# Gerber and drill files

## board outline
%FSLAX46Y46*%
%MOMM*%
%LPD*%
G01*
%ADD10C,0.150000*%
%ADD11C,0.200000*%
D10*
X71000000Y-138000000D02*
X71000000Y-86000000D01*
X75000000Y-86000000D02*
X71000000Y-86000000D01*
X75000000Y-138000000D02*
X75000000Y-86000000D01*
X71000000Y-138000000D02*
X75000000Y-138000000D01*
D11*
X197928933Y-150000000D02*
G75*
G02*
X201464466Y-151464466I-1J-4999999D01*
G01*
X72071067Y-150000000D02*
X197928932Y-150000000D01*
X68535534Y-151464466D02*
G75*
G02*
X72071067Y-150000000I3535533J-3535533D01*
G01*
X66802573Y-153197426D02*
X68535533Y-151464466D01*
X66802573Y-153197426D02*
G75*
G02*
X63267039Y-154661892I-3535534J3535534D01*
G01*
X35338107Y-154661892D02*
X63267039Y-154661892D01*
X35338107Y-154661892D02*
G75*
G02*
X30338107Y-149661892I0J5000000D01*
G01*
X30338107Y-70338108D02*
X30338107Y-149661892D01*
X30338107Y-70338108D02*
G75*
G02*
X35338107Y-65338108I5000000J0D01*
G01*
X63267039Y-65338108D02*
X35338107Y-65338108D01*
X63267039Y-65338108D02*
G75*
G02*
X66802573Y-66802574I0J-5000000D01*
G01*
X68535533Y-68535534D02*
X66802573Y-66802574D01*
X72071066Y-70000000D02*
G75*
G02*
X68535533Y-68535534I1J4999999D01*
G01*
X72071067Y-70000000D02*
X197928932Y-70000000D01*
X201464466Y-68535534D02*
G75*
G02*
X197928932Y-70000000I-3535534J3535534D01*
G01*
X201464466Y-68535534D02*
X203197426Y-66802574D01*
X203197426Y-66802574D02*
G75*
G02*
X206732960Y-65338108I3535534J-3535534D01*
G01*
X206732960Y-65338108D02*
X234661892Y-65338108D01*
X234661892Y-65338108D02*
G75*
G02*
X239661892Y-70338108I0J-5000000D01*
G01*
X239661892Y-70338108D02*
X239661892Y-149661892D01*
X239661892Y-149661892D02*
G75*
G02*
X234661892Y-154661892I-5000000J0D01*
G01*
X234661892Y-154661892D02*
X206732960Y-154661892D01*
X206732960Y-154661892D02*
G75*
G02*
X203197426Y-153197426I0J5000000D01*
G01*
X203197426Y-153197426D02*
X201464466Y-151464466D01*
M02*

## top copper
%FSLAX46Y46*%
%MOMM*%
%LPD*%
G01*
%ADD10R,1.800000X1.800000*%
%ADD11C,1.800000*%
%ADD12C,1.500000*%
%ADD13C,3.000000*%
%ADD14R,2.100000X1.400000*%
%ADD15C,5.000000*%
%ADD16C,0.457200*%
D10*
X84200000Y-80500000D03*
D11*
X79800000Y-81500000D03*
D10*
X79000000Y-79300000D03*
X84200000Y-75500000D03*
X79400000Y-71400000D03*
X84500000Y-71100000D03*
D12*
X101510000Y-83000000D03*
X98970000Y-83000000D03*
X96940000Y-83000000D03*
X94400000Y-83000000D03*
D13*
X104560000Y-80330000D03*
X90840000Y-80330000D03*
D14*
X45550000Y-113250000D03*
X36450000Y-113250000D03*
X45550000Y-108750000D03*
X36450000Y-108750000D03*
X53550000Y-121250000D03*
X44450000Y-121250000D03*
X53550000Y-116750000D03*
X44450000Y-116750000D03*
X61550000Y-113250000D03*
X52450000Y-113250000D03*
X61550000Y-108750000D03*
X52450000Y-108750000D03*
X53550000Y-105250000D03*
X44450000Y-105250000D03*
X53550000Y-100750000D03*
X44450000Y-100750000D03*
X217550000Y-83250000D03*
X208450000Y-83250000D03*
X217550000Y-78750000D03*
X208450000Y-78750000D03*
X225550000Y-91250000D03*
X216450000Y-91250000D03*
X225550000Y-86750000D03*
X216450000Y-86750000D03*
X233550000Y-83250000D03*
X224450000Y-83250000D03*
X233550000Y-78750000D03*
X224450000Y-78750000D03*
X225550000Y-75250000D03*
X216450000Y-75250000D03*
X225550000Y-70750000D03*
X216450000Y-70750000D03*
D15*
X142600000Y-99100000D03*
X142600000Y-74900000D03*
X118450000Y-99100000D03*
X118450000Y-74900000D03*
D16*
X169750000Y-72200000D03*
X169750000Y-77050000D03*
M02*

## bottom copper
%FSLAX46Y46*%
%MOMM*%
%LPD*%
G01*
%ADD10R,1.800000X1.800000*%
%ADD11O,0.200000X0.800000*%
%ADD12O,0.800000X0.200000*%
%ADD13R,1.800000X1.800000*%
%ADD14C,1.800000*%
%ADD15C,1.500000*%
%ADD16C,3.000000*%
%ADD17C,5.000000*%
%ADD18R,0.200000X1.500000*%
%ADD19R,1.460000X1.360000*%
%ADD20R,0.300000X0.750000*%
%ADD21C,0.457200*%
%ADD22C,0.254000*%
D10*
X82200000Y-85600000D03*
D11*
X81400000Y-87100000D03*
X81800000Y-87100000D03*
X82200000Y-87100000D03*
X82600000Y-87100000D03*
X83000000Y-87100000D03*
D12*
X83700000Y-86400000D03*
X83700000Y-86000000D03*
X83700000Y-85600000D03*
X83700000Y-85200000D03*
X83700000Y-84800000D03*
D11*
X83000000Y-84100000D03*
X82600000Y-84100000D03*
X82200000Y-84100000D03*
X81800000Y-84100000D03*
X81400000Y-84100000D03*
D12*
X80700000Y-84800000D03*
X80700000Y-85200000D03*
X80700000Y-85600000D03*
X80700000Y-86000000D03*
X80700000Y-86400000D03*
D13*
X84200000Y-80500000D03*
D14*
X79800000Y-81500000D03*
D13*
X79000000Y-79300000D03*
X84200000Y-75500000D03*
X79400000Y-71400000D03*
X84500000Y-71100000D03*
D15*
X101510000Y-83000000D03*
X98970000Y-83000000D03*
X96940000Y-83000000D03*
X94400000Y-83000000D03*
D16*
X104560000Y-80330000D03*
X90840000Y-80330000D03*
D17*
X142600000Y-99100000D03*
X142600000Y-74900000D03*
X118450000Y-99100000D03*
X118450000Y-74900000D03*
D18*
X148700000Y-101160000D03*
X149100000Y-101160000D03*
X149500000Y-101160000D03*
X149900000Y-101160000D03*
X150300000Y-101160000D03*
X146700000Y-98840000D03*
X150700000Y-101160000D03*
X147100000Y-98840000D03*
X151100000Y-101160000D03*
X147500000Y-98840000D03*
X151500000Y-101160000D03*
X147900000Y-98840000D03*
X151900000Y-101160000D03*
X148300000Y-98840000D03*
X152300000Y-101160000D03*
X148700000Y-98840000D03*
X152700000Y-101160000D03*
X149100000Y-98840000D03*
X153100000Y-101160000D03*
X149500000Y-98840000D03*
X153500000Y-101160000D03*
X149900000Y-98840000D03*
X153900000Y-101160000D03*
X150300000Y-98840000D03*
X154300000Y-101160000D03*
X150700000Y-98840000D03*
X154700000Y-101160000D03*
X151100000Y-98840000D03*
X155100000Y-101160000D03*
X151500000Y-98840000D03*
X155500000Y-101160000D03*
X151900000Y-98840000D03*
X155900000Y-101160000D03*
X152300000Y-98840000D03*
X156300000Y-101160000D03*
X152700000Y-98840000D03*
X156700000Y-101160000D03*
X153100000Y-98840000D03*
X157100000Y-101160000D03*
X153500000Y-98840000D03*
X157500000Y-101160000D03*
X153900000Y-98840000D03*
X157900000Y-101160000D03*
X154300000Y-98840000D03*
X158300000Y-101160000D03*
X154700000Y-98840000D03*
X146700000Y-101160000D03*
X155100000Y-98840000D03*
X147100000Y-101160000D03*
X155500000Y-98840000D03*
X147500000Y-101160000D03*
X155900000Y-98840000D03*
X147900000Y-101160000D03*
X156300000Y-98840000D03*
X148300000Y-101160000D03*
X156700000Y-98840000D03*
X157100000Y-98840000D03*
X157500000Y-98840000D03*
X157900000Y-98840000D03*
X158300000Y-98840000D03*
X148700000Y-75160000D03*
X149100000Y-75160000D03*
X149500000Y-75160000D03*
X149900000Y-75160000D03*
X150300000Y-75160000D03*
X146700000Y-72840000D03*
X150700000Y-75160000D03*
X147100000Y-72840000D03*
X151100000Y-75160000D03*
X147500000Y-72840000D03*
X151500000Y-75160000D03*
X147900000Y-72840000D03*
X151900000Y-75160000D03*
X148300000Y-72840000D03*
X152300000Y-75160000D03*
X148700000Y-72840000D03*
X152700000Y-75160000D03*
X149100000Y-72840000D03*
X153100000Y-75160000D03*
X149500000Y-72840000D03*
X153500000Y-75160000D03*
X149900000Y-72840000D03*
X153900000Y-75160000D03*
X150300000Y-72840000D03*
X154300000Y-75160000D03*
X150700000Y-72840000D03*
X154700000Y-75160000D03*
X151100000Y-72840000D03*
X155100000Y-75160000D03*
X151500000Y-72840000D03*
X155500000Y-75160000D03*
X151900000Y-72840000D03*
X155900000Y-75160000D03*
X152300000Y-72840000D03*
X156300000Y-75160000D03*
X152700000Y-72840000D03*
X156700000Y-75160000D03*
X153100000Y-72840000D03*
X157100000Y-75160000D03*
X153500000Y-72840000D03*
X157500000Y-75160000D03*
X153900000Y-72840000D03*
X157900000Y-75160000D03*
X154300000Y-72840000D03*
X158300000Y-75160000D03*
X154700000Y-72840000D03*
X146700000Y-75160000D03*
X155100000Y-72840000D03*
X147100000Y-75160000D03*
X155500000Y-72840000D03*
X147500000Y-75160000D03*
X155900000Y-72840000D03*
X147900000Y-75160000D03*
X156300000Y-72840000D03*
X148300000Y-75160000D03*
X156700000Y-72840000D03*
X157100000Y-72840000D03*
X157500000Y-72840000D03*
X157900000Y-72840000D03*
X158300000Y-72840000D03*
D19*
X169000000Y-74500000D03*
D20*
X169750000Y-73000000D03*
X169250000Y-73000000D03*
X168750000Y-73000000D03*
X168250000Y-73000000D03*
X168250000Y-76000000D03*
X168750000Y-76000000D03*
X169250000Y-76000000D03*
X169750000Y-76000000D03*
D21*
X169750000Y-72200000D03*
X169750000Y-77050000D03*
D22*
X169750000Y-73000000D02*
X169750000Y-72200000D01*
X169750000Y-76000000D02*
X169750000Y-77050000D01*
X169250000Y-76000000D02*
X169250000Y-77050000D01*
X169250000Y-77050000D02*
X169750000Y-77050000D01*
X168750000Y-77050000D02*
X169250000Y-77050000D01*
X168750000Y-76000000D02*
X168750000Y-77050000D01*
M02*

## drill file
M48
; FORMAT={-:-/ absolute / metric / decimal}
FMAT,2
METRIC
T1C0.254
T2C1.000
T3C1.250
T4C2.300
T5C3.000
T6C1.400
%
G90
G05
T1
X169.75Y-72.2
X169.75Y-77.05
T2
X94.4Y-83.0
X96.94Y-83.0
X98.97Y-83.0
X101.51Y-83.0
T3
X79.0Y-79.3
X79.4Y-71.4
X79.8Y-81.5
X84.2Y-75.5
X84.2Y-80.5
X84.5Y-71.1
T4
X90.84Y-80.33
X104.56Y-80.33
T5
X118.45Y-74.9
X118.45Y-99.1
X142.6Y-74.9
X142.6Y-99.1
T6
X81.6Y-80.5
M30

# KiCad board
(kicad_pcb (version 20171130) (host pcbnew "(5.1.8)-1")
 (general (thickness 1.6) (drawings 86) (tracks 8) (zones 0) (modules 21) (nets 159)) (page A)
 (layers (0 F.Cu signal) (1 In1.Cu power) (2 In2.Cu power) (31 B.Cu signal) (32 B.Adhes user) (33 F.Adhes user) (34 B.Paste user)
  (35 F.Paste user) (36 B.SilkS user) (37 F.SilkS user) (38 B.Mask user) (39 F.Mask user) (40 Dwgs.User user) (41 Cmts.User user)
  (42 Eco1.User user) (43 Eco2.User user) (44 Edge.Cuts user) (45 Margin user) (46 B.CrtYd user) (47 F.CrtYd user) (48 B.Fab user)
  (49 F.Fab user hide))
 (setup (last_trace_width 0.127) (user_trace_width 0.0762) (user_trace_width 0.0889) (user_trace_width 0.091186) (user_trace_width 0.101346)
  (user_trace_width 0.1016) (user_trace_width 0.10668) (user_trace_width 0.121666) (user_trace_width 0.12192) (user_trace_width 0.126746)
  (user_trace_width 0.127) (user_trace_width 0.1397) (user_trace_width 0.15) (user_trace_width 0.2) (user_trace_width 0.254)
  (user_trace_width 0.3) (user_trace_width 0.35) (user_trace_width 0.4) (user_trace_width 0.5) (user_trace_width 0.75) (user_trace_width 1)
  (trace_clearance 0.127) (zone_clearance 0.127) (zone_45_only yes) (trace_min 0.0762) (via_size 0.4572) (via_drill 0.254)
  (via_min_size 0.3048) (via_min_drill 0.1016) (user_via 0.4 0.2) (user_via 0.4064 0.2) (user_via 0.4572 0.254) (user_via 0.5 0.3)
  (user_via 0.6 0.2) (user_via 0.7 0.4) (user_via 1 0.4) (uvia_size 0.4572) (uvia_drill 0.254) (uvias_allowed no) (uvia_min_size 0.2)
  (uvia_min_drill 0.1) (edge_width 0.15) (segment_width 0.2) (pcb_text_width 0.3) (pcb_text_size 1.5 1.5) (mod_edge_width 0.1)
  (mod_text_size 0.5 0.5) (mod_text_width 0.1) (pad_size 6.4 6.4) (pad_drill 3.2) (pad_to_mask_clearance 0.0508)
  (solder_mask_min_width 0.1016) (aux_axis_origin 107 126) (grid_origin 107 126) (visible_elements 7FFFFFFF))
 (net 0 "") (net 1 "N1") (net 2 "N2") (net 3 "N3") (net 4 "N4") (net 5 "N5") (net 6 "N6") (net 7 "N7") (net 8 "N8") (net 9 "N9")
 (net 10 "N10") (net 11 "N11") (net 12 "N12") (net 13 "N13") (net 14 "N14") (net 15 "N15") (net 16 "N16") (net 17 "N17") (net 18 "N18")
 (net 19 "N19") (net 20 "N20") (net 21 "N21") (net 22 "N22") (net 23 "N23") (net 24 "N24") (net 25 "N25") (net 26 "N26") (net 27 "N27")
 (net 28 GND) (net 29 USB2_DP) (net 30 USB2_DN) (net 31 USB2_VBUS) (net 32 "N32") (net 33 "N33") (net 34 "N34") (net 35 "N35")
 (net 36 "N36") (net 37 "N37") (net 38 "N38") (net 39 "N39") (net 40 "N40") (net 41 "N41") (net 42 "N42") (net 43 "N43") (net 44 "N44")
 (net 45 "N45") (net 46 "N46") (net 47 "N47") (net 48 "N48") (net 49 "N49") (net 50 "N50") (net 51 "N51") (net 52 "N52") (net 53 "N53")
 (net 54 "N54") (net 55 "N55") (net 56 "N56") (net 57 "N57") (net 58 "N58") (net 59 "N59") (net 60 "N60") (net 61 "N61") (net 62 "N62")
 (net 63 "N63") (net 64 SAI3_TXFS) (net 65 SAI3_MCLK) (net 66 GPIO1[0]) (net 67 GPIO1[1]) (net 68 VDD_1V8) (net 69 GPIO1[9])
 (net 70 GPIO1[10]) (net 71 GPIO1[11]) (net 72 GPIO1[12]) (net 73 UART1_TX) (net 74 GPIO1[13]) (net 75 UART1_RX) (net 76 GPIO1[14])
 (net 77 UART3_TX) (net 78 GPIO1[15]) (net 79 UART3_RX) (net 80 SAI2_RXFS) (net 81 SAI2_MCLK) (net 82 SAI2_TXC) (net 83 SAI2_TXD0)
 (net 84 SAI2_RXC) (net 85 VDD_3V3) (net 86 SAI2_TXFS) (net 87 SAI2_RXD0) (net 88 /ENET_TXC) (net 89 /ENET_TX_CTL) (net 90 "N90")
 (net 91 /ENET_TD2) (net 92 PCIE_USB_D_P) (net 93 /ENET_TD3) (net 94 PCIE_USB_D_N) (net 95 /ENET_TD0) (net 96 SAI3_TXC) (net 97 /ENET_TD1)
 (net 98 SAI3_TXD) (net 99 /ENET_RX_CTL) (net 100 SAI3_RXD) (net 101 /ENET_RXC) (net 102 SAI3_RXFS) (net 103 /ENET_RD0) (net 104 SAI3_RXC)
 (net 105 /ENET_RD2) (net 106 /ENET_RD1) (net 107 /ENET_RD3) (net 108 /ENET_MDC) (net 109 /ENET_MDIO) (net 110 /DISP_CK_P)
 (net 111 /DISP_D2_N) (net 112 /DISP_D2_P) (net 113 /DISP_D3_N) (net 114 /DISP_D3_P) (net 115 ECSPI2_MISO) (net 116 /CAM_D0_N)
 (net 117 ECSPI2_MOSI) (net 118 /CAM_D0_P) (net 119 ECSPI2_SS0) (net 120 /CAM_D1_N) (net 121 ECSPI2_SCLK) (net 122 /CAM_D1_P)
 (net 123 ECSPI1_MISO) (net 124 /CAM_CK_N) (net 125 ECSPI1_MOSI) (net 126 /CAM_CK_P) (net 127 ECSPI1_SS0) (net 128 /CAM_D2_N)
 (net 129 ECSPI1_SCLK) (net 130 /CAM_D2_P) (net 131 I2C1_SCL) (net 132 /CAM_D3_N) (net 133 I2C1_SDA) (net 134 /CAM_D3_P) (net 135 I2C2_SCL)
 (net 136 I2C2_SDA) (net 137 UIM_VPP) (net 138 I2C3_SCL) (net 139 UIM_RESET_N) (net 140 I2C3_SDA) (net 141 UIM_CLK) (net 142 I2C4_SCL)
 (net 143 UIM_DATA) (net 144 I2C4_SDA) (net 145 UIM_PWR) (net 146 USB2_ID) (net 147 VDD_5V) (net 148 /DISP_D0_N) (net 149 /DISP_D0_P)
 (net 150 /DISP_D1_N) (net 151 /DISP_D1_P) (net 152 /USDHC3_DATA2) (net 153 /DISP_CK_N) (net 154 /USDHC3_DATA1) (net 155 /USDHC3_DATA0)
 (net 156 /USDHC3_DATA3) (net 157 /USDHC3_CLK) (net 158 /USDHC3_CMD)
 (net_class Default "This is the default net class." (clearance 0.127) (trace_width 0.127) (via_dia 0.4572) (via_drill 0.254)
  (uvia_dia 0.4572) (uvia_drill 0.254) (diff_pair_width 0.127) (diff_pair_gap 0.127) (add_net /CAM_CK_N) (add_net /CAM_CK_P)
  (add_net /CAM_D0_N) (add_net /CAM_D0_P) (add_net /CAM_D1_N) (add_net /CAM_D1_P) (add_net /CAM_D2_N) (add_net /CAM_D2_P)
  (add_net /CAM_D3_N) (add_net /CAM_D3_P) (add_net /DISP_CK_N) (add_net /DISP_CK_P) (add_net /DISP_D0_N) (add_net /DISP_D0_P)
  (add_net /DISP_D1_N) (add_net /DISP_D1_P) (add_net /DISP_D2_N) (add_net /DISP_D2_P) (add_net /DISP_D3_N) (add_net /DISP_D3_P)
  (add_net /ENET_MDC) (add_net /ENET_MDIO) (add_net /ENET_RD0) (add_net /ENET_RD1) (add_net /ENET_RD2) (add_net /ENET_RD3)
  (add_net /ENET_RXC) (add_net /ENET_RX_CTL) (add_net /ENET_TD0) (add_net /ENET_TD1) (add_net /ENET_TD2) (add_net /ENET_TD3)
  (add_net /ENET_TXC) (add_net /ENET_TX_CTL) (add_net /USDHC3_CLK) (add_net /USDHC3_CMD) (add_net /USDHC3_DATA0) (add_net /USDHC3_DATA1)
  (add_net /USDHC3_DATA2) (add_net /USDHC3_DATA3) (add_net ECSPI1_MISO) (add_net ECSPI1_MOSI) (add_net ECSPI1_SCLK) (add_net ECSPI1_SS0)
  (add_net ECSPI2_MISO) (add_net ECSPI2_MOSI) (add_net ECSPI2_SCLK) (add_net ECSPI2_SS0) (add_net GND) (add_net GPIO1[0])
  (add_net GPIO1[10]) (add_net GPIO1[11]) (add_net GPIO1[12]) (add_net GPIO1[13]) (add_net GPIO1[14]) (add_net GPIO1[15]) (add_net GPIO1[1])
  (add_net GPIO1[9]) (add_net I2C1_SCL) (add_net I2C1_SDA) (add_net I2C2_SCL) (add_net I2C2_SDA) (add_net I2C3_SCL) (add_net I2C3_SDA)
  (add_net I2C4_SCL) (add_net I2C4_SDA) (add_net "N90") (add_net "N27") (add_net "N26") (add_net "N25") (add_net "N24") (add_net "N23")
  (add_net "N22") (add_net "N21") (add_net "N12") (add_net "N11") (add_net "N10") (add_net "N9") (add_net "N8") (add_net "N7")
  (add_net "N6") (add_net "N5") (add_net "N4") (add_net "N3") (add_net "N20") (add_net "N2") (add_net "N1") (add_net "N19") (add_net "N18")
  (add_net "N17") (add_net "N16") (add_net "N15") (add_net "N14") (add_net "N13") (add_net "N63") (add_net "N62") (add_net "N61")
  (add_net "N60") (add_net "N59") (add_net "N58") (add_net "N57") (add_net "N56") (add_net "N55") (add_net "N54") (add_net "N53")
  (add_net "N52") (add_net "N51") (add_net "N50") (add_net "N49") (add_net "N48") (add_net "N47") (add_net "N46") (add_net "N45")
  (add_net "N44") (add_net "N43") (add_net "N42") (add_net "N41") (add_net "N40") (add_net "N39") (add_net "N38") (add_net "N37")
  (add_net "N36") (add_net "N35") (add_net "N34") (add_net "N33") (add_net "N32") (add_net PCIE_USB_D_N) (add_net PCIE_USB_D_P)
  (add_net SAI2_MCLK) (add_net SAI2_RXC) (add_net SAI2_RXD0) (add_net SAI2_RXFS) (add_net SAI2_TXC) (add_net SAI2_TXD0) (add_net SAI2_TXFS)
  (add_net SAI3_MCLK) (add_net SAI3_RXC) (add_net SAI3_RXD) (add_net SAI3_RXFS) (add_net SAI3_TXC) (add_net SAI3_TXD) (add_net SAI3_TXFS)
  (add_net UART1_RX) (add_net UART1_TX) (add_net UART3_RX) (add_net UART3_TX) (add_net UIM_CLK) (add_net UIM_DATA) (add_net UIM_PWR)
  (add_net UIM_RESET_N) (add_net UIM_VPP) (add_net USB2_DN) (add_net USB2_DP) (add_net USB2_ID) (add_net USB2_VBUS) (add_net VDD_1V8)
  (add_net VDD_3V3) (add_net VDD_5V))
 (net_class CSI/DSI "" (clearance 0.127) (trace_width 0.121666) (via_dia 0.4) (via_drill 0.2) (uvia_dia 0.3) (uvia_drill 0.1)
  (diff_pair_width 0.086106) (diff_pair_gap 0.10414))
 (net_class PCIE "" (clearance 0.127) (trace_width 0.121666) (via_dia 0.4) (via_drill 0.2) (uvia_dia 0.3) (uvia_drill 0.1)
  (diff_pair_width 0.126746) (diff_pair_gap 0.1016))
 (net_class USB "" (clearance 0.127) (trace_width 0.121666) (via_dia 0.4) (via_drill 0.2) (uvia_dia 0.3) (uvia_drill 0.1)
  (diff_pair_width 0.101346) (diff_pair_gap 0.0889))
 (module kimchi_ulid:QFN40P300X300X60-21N (layer B.Cu) (at 82.2 85.6)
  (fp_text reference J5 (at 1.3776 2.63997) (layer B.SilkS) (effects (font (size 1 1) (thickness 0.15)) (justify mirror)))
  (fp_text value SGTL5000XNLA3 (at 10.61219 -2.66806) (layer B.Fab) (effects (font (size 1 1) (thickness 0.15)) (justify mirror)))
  (pad 21 smd rect (at 0 0) (size 1.8 1.8) (layers B.Cu B.Mask) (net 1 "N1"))
  (pad 20 smd oval (at -0.8 1.5) (size 0.2 0.8) (layers B.Cu B.Paste B.Mask) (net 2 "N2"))
  (pad 19 smd oval (at -0.4 1.5) (size 0.2 0.8) (layers B.Cu B.Paste B.Mask) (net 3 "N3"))
  (pad 18 smd oval (at 0 1.5) (size 0.2 0.8) (layers B.Cu B.Paste B.Mask) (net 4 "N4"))
  (pad 17 smd oval (at 0.4 1.5) (size 0.2 0.8) (layers B.Cu B.Paste B.Mask) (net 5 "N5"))
  (pad 16 smd oval (at 0.8 1.5) (size 0.2 0.8) (layers B.Cu B.Paste B.Mask) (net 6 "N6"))
  (pad 15 smd oval (at 1.5 0.8) (size 0.8 0.2) (layers B.Cu B.Paste B.Mask) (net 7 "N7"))
  (pad 14 smd oval (at 1.5 0.4) (size 0.8 0.2) (layers B.Cu B.Paste B.Mask) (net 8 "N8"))
  (pad 13 smd oval (at 1.5 0) (size 0.8 0.2) (layers B.Cu B.Paste B.Mask) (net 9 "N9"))
  (pad 12 smd oval (at 1.5 -0.4) (size 0.8 0.2) (layers B.Cu B.Paste B.Mask) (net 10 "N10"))
  (pad 11 smd oval (at 1.5 -0.8) (size 0.8 0.2) (layers B.Cu B.Paste B.Mask) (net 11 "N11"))
  (pad 10 smd oval (at 0.8 -1.5) (size 0.2 0.8) (layers B.Cu B.Paste B.Mask) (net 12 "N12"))
  (pad 9 smd oval (at 0.4 -1.5) (size 0.2 0.8) (layers B.Cu B.Paste B.Mask) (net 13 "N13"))
  (pad 8 smd oval (at 0 -1.5) (size 0.2 0.8) (layers B.Cu B.Paste B.Mask) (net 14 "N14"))
  (pad 7 smd oval (at -0.4 -1.5) (size 0.2 0.8) (layers B.Cu B.Paste B.Mask) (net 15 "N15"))
  (pad 6 smd oval (at -0.8 -1.5) (size 0.2 0.8) (layers B.Cu B.Paste B.Mask) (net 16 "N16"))
  (pad 5 smd oval (at -1.5 -0.8) (size 0.8 0.2) (layers B.Cu B.Paste B.Mask) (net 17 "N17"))
  (pad 4 smd oval (at -1.5 -0.4) (size 0.8 0.2) (layers B.Cu B.Paste B.Mask) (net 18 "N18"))
  (pad 3 smd oval (at -1.5 0) (size 0.8 0.2) (layers B.Cu B.Paste B.Mask) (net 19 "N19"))
  (pad 2 smd oval (at -1.5 0.4) (size 0.8 0.2) (layers B.Cu B.Paste B.Mask) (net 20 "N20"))
  (pad 1 smd oval (at -1.5 0.8) (size 0.8 0.2) (layers B.Cu B.Paste B.Mask) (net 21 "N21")))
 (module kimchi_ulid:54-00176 (layer B.Cu) (at 81.6 70 270)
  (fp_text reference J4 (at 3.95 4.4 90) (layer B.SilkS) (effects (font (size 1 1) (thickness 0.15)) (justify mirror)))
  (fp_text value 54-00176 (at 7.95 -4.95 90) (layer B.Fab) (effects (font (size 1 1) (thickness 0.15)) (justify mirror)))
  (pad "" np_thru_hole circle (at 10.5 0 270) (size 1.4 1.4) (drill 1.4) (layers *.Cu *.Mask))
  (pad 6 thru_hole rect (at 10.5 -2.6 270) (size 1.8 1.8) (drill 1.25) (layers *.Cu *.Mask) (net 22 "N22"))
  (pad 5 thru_hole circle (at 11.5 1.8 270) (size 1.8 1.8) (drill 1.25) (layers *.Cu *.Mask) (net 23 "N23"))
  (pad 4 thru_hole rect (at 9.3 2.6 270) (size 1.8 1.8) (drill 1.25) (layers *.Cu *.Mask) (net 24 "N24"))
  (pad 3 thru_hole rect (at 5.5 -2.6 270) (size 1.8 1.8) (drill 1.25) (layers *.Cu *.Mask) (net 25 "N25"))
  (pad 2 thru_hole rect (at 1.4 2.2 270) (size 1.8 1.8) (drill 1.25) (layers *.Cu *.Mask) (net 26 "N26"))
  (pad 1 thru_hole rect (at 1.1 -2.9 270) (size 1.8 1.8) (drill 1.25) (layers *.Cu *.Mask) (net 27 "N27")))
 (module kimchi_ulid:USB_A (layer B.Cu) (at 94.4 83)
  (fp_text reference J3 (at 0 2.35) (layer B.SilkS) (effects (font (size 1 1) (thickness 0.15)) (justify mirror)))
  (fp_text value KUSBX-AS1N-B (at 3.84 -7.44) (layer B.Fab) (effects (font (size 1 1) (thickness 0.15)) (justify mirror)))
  (pad 4 thru_hole circle (at 7.11 0 90) (size 1.5 1.5) (drill 1) (layers *.Cu *.Mask) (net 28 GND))
  (pad 3 thru_hole circle (at 4.57 0 90) (size 1.5 1.5) (drill 1) (layers *.Cu *.Mask) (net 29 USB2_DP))
  (pad 2 thru_hole circle (at 2.54 0 90) (size 1.5 1.5) (drill 1) (layers *.Cu *.Mask) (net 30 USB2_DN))
  (pad 1 thru_hole circle (at 0 0 90) (size 1.5 1.5) (drill 1) (layers *.Cu *.Mask) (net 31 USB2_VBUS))
  (pad 5 thru_hole circle (at 10.16 -2.67 90) (size 3 3) (drill 2.3) (layers *.Cu *.Mask) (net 28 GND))
  (pad 5 thru_hole circle (at -3.56 -2.67 90) (size 3 3) (drill 2.3) (layers *.Cu *.Mask) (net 28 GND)))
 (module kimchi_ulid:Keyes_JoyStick (layer F.Cu) (at 221 111 180)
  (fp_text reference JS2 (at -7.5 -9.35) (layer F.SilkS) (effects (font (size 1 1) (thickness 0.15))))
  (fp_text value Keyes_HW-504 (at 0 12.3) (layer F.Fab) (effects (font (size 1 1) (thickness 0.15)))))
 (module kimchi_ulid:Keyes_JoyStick (layer F.Cu) (at 48.8 81)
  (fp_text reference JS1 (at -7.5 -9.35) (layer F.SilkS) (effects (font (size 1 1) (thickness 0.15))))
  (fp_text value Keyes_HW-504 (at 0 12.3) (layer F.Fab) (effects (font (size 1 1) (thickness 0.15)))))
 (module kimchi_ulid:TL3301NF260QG (layer F.Cu) (at 41 111)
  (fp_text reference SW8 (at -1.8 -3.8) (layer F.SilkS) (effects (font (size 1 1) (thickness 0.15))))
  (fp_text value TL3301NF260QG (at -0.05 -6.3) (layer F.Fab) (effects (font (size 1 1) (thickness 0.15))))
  (pad 4 smd rect (at 4.55 2.25) (size 2.1 1.4) (layers F.Cu F.Paste F.Mask) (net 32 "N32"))
  (pad 3 smd rect (at -4.55 2.25) (size 2.1 1.4) (layers F.Cu F.Paste F.Mask) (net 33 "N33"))
  (pad 2 smd rect (at 4.55 -2.25) (size 2.1 1.4) (layers F.Cu F.Paste F.Mask) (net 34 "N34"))
  (pad 1 smd rect (at -4.55 -2.25) (size 2.1 1.4) (layers F.Cu F.Paste F.Mask) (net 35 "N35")))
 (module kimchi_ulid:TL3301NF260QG (layer F.Cu) (at 49 119)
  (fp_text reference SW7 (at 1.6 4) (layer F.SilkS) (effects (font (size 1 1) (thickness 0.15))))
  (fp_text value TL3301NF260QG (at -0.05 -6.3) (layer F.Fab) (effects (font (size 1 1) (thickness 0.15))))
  (pad 4 smd rect (at 4.55 2.25) (size 2.1 1.4) (layers F.Cu F.Paste F.Mask) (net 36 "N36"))
  (pad 3 smd rect (at -4.55 2.25) (size 2.1 1.4) (layers F.Cu F.Paste F.Mask) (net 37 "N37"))
  (pad 2 smd rect (at 4.55 -2.25) (size 2.1 1.4) (layers F.Cu F.Paste F.Mask) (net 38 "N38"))
  (pad 1 smd rect (at -4.55 -2.25) (size 2.1 1.4) (layers F.Cu F.Paste F.Mask) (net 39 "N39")))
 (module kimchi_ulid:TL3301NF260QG (layer F.Cu) (at 57 111)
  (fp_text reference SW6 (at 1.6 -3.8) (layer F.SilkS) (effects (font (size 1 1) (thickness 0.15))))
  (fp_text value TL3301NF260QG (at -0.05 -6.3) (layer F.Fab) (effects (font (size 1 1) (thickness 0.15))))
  (pad 4 smd rect (at 4.55 2.25) (size 2.1 1.4) (layers F.Cu F.Paste F.Mask) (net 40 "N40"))
  (pad 3 smd rect (at -4.55 2.25) (size 2.1 1.4) (layers F.Cu F.Paste F.Mask) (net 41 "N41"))
  (pad 2 smd rect (at 4.55 -2.25) (size 2.1 1.4) (layers F.Cu F.Paste F.Mask) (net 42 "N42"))
  (pad 1 smd rect (at -4.55 -2.25) (size 2.1 1.4) (layers F.Cu F.Paste F.Mask) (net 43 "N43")))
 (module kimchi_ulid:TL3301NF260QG (layer F.Cu) (at 49 103)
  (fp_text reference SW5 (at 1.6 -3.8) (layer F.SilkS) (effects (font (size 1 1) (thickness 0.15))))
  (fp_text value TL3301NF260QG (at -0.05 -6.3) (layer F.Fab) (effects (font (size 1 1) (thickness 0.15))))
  (pad 4 smd rect (at 4.55 2.25) (size 2.1 1.4) (layers F.Cu F.Paste F.Mask) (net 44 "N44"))
  (pad 3 smd rect (at -4.55 2.25) (size 2.1 1.4) (layers F.Cu F.Paste F.Mask) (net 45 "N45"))
  (pad 2 smd rect (at 4.55 -2.25) (size 2.1 1.4) (layers F.Cu F.Paste F.Mask) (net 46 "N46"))
  (pad 1 smd rect (at -4.55 -2.25) (size 2.1 1.4) (layers F.Cu F.Paste F.Mask) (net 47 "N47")))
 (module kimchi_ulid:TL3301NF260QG (layer F.Cu) (at 213 81)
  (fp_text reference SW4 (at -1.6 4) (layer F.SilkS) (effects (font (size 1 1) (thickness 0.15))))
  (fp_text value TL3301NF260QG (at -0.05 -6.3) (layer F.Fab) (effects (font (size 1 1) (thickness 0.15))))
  (pad 4 smd rect (at 4.55 2.25) (size 2.1 1.4) (layers F.Cu F.Paste F.Mask) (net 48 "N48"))
  (pad 3 smd rect (at -4.55 2.25) (size 2.1 1.4) (layers F.Cu F.Paste F.Mask) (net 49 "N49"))
  (pad 2 smd rect (at 4.55 -2.25) (size 2.1 1.4) (layers F.Cu F.Paste F.Mask) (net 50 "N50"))
  (pad 1 smd rect (at -4.55 -2.25) (size 2.1 1.4) (layers F.Cu F.Paste F.Mask) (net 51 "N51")))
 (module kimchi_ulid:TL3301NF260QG (layer F.Cu) (at 221 89)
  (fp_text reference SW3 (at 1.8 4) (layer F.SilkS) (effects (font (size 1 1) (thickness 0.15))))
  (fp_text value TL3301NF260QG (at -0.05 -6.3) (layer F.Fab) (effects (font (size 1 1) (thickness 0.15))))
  (pad 4 smd rect (at 4.55 2.25) (size 2.1 1.4) (layers F.Cu F.Paste F.Mask) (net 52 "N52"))
  (pad 3 smd rect (at -4.55 2.25) (size 2.1 1.4) (layers F.Cu F.Paste F.Mask) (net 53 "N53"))
  (pad 2 smd rect (at 4.55 -2.25) (size 2.1 1.4) (layers F.Cu F.Paste F.Mask) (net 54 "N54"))
  (pad 1 smd rect (at -4.55 -2.25) (size 2.1 1.4) (layers F.Cu F.Paste F.Mask) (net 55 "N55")))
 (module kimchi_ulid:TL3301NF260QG (layer F.Cu) (at 229 81)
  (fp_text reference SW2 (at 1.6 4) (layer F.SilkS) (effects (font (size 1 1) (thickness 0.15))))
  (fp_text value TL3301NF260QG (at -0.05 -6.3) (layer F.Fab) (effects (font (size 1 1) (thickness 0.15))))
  (pad 4 smd rect (at 4.55 2.25) (size 2.1 1.4) (layers F.Cu F.Paste F.Mask) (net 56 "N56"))
  (pad 3 smd rect (at -4.55 2.25) (size 2.1 1.4) (layers F.Cu F.Paste F.Mask) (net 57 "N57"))
  (pad 2 smd rect (at 4.55 -2.25) (size 2.1 1.4) (layers F.Cu F.Paste F.Mask) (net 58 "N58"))
  (pad 1 smd rect (at -4.55 -2.25) (size 2.1 1.4) (layers F.Cu F.Paste F.Mask) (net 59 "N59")))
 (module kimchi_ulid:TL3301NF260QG (layer F.Cu) (at 221 73)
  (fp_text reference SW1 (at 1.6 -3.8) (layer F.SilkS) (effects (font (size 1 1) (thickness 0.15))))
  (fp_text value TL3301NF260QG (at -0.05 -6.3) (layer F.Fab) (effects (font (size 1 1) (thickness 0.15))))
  (pad 4 smd rect (at 4.55 2.25) (size 2.1 1.4) (layers F.Cu F.Paste F.Mask) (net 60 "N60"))
  (pad 3 smd rect (at -4.55 2.25) (size 2.1 1.4) (layers F.Cu F.Paste F.Mask) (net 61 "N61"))
  (pad 2 smd rect (at 4.55 -2.25) (size 2.1 1.4) (layers F.Cu F.Paste F.Mask) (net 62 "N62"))
  (pad 1 smd rect (at -4.55 -2.25) (size 2.1 1.4) (layers F.Cu F.Paste F.Mask) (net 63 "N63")))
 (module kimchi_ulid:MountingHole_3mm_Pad (layer F.Cu) (at 142.6 99.1)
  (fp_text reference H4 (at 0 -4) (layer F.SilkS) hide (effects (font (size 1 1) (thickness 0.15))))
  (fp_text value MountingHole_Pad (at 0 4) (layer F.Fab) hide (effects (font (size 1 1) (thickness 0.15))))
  (pad 1 thru_hole circle (at 0 0) (size 5 5) (drill 3) (layers *.Cu *.Mask) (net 28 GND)))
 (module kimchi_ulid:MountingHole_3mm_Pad (layer F.Cu) (at 142.6 74.9)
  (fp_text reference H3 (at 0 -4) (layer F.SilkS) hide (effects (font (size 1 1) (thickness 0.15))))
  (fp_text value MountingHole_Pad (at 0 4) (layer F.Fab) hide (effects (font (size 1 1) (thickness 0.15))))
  (pad 1 thru_hole circle (at 0 0) (size 5 5) (drill 3) (layers *.Cu *.Mask) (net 28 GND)))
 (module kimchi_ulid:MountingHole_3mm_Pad (layer F.Cu) (at 118.45 99.1)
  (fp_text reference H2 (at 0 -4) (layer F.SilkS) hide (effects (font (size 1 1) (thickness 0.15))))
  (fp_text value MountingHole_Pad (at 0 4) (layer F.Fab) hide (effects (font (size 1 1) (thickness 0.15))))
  (pad 1 thru_hole circle (at 0 0) (size 5 5) (drill 3) (layers *.Cu *.Mask) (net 28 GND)))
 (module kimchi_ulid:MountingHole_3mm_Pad (layer F.Cu) (at 118.45 74.9)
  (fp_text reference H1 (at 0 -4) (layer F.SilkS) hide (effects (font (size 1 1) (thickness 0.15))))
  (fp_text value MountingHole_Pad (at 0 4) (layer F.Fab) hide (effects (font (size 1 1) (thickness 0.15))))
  (pad 1 thru_hole circle (at 0 0) (size 5 5) (drill 3) (layers *.Cu *.Mask) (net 28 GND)))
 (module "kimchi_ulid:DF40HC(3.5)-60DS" (layer B.Cu) (at 152.5 100 180)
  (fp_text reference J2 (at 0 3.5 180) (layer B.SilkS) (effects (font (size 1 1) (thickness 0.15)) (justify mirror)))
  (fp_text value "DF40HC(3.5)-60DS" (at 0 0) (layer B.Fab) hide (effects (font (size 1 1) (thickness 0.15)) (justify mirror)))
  (pad 36 smd rect (at 3.8 -1.16 180) (size 0.2 1.5) (layers B.Cu B.Paste B.Mask) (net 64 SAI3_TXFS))
  (pad 37 smd rect (at 3.4 -1.16 180) (size 0.2 1.5) (layers B.Cu B.Paste B.Mask) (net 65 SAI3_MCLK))
  (pad 38 smd rect (at 3 -1.16 180) (size 0.2 1.5) (layers B.Cu B.Paste B.Mask) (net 28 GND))
  (pad 39 smd rect (at 2.6 -1.16 180) (size 0.2 1.5) (layers B.Cu B.Paste B.Mask) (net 28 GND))
  (pad 40 smd rect (at 2.2 -1.16 180) (size 0.2 1.5) (layers B.Cu B.Paste B.Mask) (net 28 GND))
  (pad 30 smd rect (at 5.8 1.16 180) (size 0.2 1.5) (layers B.Cu B.Paste B.Mask) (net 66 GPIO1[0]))
  (pad 41 smd rect (at 1.8 -1.16 180) (size 0.2 1.5) (layers B.Cu B.Paste B.Mask) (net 28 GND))
  (pad 29 smd rect (at 5.4 1.16 180) (size 0.2 1.5) (layers B.Cu B.Paste B.Mask) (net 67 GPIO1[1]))
  (pad 42 smd rect (at 1.4 -1.16 180) (size 0.2 1.5) (layers B.Cu B.Paste B.Mask) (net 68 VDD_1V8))
  (pad 28 smd rect (at 5 1.16 180) (size 0.2 1.5) (layers B.Cu B.Paste B.Mask) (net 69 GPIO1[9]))
  (pad 43 smd rect (at 1 -1.16 180) (size 0.2 1.5) (layers B.Cu B.Paste B.Mask) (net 68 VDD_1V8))
  (pad 27 smd rect (at 4.6 1.16 180) (size 0.2 1.5) (layers B.Cu B.Paste B.Mask) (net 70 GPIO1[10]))
  (pad 44 smd rect (at 0.6 -1.16 180) (size 0.2 1.5) (layers B.Cu B.Paste B.Mask) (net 68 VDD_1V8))
  (pad 26 smd rect (at 4.2 1.16 180) (size 0.2 1.5) (layers B.Cu B.Paste B.Mask) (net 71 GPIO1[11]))
  (pad 45 smd rect (at 0.2 -1.16 180) (size 0.2 1.5) (layers B.Cu B.Paste B.Mask) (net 68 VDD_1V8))
  (pad 25 smd rect (at 3.8 1.16 180) (size 0.2 1.5) (layers B.Cu B.Paste B.Mask) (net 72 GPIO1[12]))
  (pad 46 smd rect (at -0.2 -1.16 180) (size 0.2 1.5) (layers B.Cu B.Paste B.Mask) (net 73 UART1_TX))
  (pad 24 smd rect (at 3.4 1.16 180) (size 0.2 1.5) (layers B.Cu B.Paste B.Mask) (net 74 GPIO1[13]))
  (pad 47 smd rect (at -0.6 -1.16 180) (size 0.2 1.5) (layers B.Cu B.Paste B.Mask) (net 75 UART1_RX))
  (pad 23 smd rect (at 3 1.16 180) (size 0.2 1.5) (layers B.Cu B.Paste B.Mask) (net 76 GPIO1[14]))
  (pad 48 smd rect (at -1 -1.16 180) (size 0.2 1.5) (layers B.Cu B.Paste B.Mask) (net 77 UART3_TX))
  (pad 22 smd rect (at 2.6 1.16 180) (size 0.2 1.5) (layers B.Cu B.Paste B.Mask) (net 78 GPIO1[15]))
  (pad 49 smd rect (at -1.4 -1.16 180) (size 0.2 1.5) (layers B.Cu B.Paste B.Mask) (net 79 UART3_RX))
  (pad 21 smd rect (at 2.2 1.16 180) (size 0.2 1.5) (layers B.Cu B.Paste B.Mask) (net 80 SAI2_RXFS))
  (pad 50 smd rect (at -1.8 -1.16 180) (size 0.2 1.5) (layers B.Cu B.Paste B.Mask) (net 28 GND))
  (pad 20 smd rect (at 1.8 1.16 180) (size 0.2 1.5) (layers B.Cu B.Paste B.Mask) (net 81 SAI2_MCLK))
  (pad 51 smd rect (at -2.2 -1.16 180) (size 0.2 1.5) (layers B.Cu B.Paste B.Mask) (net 28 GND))
  (pad 19 smd rect (at 1.4 1.16 180) (size 0.2 1.5) (layers B.Cu B.Paste B.Mask) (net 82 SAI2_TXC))
  (pad 52 smd rect (at -2.6 -1.16 180) (size 0.2 1.5) (layers B.Cu B.Paste B.Mask) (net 28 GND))
  (pad 18 smd rect (at 1 1.16 180) (size 0.2 1.5) (layers B.Cu B.Paste B.Mask) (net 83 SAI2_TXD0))
  (pad 53 smd rect (at -3 -1.16 180) (size 0.2 1.5) (layers B.Cu B.Paste B.Mask) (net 28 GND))
  (pad 17 smd rect (at 0.6 1.16 180) (size 0.2 1.5) (layers B.Cu B.Paste B.Mask) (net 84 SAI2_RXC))
  (pad 54 smd rect (at -3.4 -1.16 180) (size 0.2 1.5) (layers B.Cu B.Paste B.Mask) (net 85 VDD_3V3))
  (pad 16 smd rect (at 0.2 1.16 180) (size 0.2 1.5) (layers B.Cu B.Paste B.Mask) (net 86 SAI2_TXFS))
  (pad 55 smd rect (at -3.8 -1.16 180) (size 0.2 1.5) (layers B.Cu B.Paste B.Mask) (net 85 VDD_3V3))
  (pad 15 smd rect (at -0.2 1.16 180) (size 0.2 1.5) (layers B.Cu B.Paste B.Mask) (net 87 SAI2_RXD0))
  (pad 56 smd rect (at -4.2 -1.16 180) (size 0.2 1.5) (layers B.Cu B.Paste B.Mask) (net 85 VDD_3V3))
  (pad 14 smd rect (at -0.6 1.16 180) (size 0.2 1.5) (layers B.Cu B.Paste B.Mask) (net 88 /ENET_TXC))
  (pad 57 smd rect (at -4.6 -1.16 180) (size 0.2 1.5) (layers B.Cu B.Paste B.Mask) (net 85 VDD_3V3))
  (pad 13 smd rect (at -1 1.16 180) (size 0.2 1.5) (layers B.Cu B.Paste B.Mask) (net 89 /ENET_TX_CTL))
  (pad 58 smd rect (at -5 -1.16 180) (size 0.2 1.5) (layers B.Cu B.Paste B.Mask) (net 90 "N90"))
  (pad 12 smd rect (at -1.4 1.16 180) (size 0.2 1.5) (layers B.Cu B.Paste B.Mask) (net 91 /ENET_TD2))
  (pad 59 smd rect (at -5.4 -1.16 180) (size 0.2 1.5) (layers B.Cu B.Paste B.Mask) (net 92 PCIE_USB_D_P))
  (pad 11 smd rect (at -1.8 1.16 180) (size 0.2 1.5) (layers B.Cu B.Paste B.Mask) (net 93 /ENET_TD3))
  (pad 60 smd rect (at -5.8 -1.16 180) (size 0.2 1.5) (layers B.Cu B.Paste B.Mask) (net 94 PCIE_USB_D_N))
  (pad 10 smd rect (at -2.2 1.16 180) (size 0.2 1.5) (layers B.Cu B.Paste B.Mask) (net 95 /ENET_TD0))
  (pad 31 smd rect (at 5.8 -1.16 180) (size 0.2 1.5) (layers B.Cu B.Paste B.Mask) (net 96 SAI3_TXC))
  (pad 9 smd rect (at -2.6 1.16 180) (size 0.2 1.5) (layers B.Cu B.Paste B.Mask) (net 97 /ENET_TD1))
  (pad 32 smd rect (at 5.4 -1.16 180) (size 0.2 1.5) (layers B.Cu B.Paste B.Mask) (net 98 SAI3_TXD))
  (pad 8 smd rect (at -3 1.16 180) (size 0.2 1.5) (layers B.Cu B.Paste B.Mask) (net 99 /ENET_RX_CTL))
  (pad 33 smd rect (at 5 -1.16 180) (size 0.2 1.5) (layers B.Cu B.Paste B.Mask) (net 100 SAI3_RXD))
  (pad 7 smd rect (at -3.4 1.16 180) (size 0.2 1.5) (layers B.Cu B.Paste B.Mask) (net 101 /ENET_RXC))
  (pad 34 smd rect (at 4.6 -1.16 180) (size 0.2 1.5) (layers B.Cu B.Paste B.Mask) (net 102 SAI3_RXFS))
  (pad 6 smd rect (at -3.8 1.16 180) (size 0.2 1.5) (layers B.Cu B.Paste B.Mask) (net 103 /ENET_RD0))
  (pad 35 smd rect (at 4.2 -1.16 180) (size 0.2 1.5) (layers B.Cu B.Paste B.Mask) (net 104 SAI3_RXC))
  (pad 5 smd rect (at -4.2 1.16 180) (size 0.2 1.5) (layers B.Cu B.Paste B.Mask) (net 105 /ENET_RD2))
  (pad 4 smd rect (at -4.6 1.16 180) (size 0.2 1.5) (layers B.Cu B.Paste B.Mask) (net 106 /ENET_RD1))
  (pad 3 smd rect (at -5 1.16 180) (size 0.2 1.5) (layers B.Cu B.Paste B.Mask) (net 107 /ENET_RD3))
  (pad 2 smd rect (at -5.4 1.16 180) (size 0.2 1.5) (layers B.Cu B.Paste B.Mask) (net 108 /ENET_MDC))
  (pad 1 smd rect (at -5.8 1.16 180) (size 0.2 1.5) (layers B.Cu B.Paste B.Mask) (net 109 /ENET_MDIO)))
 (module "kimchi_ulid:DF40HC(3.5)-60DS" (layer B.Cu) (at 152.5 74 180)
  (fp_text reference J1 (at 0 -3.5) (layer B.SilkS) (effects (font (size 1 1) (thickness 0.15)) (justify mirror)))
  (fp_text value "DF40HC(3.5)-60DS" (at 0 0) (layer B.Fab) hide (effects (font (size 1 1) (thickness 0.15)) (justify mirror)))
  (pad 36 smd rect (at 3.8 -1.16 180) (size 0.2 1.5) (layers B.Cu B.Paste B.Mask) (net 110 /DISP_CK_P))
  (pad 37 smd rect (at 3.4 -1.16 180) (size 0.2 1.5) (layers B.Cu B.Paste B.Mask) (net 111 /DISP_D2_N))
  (pad 38 smd rect (at 3 -1.16 180) (size 0.2 1.5) (layers B.Cu B.Paste B.Mask) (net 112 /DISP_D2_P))
  (pad 39 smd rect (at 2.6 -1.16 180) (size 0.2 1.5) (layers B.Cu B.Paste B.Mask) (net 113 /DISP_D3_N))
  (pad 40 smd rect (at 2.2 -1.16 180) (size 0.2 1.5) (layers B.Cu B.Paste B.Mask) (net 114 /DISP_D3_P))
  (pad 30 smd rect (at 5.8 1.16 180) (size 0.2 1.5) (layers B.Cu B.Paste B.Mask) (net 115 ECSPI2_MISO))
  (pad 41 smd rect (at 1.8 -1.16 180) (size 0.2 1.5) (layers B.Cu B.Paste B.Mask) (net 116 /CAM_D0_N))
  (pad 29 smd rect (at 5.4 1.16 180) (size 0.2 1.5) (layers B.Cu B.Paste B.Mask) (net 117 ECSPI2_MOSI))
  (pad 42 smd rect (at 1.4 -1.16 180) (size 0.2 1.5) (layers B.Cu B.Paste B.Mask) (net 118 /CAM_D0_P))
  (pad 28 smd rect (at 5 1.16 180) (size 0.2 1.5) (layers B.Cu B.Paste B.Mask) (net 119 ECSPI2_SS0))
  (pad 43 smd rect (at 1 -1.16 180) (size 0.2 1.5) (layers B.Cu B.Paste B.Mask) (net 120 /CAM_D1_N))
  (pad 27 smd rect (at 4.6 1.16 180) (size 0.2 1.5) (layers B.Cu B.Paste B.Mask) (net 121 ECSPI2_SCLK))
  (pad 44 smd rect (at 0.6 -1.16 180) (size 0.2 1.5) (layers B.Cu B.Paste B.Mask) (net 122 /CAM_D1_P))
  (pad 26 smd rect (at 4.2 1.16 180) (size 0.2 1.5) (layers B.Cu B.Paste B.Mask) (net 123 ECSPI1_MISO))
  (pad 45 smd rect (at 0.2 -1.16 180) (size 0.2 1.5) (layers B.Cu B.Paste B.Mask) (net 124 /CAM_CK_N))
  (pad 25 smd rect (at 3.8 1.16 180) (size 0.2 1.5) (layers B.Cu B.Paste B.Mask) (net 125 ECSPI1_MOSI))
  (pad 46 smd rect (at -0.2 -1.16 180) (size 0.2 1.5) (layers B.Cu B.Paste B.Mask) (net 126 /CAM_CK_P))
  (pad 24 smd rect (at 3.4 1.16 180) (size 0.2 1.5) (layers B.Cu B.Paste B.Mask) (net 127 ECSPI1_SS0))
  (pad 47 smd rect (at -0.6 -1.16 180) (size 0.2 1.5) (layers B.Cu B.Paste B.Mask) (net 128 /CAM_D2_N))
  (pad 23 smd rect (at 3 1.16 180) (size 0.2 1.5) (layers B.Cu B.Paste B.Mask) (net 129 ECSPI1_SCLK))
  (pad 48 smd rect (at -1 -1.16 180) (size 0.2 1.5) (layers B.Cu B.Paste B.Mask) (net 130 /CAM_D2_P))
  (pad 22 smd rect (at 2.6 1.16 180) (size 0.2 1.5) (layers B.Cu B.Paste B.Mask) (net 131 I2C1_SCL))
  (pad 49 smd rect (at -1.4 -1.16 180) (size 0.2 1.5) (layers B.Cu B.Paste B.Mask) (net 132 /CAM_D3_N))
  (pad 21 smd rect (at 2.2 1.16 180) (size 0.2 1.5) (layers B.Cu B.Paste B.Mask) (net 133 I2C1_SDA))
  (pad 50 smd rect (at -1.8 -1.16 180) (size 0.2 1.5) (layers B.Cu B.Paste B.Mask) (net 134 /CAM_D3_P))
  (pad 20 smd rect (at 1.8 1.16 180) (size 0.2 1.5) (layers B.Cu B.Paste B.Mask) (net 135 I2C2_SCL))
  (pad 51 smd rect (at -2.2 -1.16 180) (size 0.2 1.5) (layers B.Cu B.Paste B.Mask) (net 28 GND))
  (pad 19 smd rect (at 1.4 1.16 180) (size 0.2 1.5) (layers B.Cu B.Paste B.Mask) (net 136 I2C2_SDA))
  (pad 52 smd rect (at -2.6 -1.16 180) (size 0.2 1.5) (layers B.Cu B.Paste B.Mask) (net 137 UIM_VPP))
  (pad 18 smd rect (at 1 1.16 180) (size 0.2 1.5) (layers B.Cu B.Paste B.Mask) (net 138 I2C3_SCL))
  (pad 53 smd rect (at -3 -1.16 180) (size 0.2 1.5) (layers B.Cu B.Paste B.Mask) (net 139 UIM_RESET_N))
  (pad 17 smd rect (at 0.6 1.16 180) (size 0.2 1.5) (layers B.Cu B.Paste B.Mask) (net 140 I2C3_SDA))
  (pad 54 smd rect (at -3.4 -1.16 180) (size 0.2 1.5) (layers B.Cu B.Paste B.Mask) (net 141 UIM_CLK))
  (pad 16 smd rect (at 0.2 1.16 180) (size 0.2 1.5) (layers B.Cu B.Paste B.Mask) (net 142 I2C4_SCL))
  (pad 55 smd rect (at -3.8 -1.16 180) (size 0.2 1.5) (layers B.Cu B.Paste B.Mask) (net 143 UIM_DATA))
  (pad 15 smd rect (at -0.2 1.16 180) (size 0.2 1.5) (layers B.Cu B.Paste B.Mask) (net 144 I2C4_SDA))
  (pad 56 smd rect (at -4.2 -1.16 180) (size 0.2 1.5) (layers B.Cu B.Paste B.Mask) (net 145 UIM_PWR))
  (pad 14 smd rect (at -0.6 1.16 180) (size 0.2 1.5) (layers B.Cu B.Paste B.Mask) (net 28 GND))
  (pad 57 smd rect (at -4.6 -1.16 180) (size 0.2 1.5) (layers B.Cu B.Paste B.Mask) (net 31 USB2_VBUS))
  (pad 13 smd rect (at -1 1.16 180) (size 0.2 1.5) (layers B.Cu B.Paste B.Mask) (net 28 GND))
  (pad 58 smd rect (at -5 -1.16 180) (size 0.2 1.5) (layers B.Cu B.Paste B.Mask) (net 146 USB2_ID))
  (pad 12 smd rect (at -1.4 1.16 180) (size 0.2 1.5) (layers B.Cu B.Paste B.Mask) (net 28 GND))
  (pad 59 smd rect (at -5.4 -1.16 180) (size 0.2 1.5) (layers B.Cu B.Paste B.Mask) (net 30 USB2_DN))
  (pad 11 smd rect (at -1.8 1.16 180) (size 0.2 1.5) (layers B.Cu B.Paste B.Mask) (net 28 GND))
  (pad 60 smd rect (at -5.8 -1.16 180) (size 0.2 1.5) (layers B.Cu B.Paste B.Mask) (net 29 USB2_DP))
  (pad 10 smd rect (at -2.2 1.16 180) (size 0.2 1.5) (layers B.Cu B.Paste B.Mask) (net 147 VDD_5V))
  (pad 31 smd rect (at 5.8 -1.16 180) (size 0.2 1.5) (layers B.Cu B.Paste B.Mask) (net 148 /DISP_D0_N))
  (pad 9 smd rect (at -2.6 1.16 180) (size 0.2 1.5) (layers B.Cu B.Paste B.Mask) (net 147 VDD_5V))
  (pad 32 smd rect (at 5.4 -1.16 180) (size 0.2 1.5) (layers B.Cu B.Paste B.Mask) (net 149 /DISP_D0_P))
  (pad 8 smd rect (at -3 1.16 180) (size 0.2 1.5) (layers B.Cu B.Paste B.Mask) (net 147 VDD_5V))
  (pad 33 smd rect (at 5 -1.16 180) (size 0.2 1.5) (layers B.Cu B.Paste B.Mask) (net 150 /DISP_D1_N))
  (pad 7 smd rect (at -3.4 1.16 180) (size 0.2 1.5) (layers B.Cu B.Paste B.Mask) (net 147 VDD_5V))
  (pad 34 smd rect (at 4.6 -1.16 180) (size 0.2 1.5) (layers B.Cu B.Paste B.Mask) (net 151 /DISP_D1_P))
  (pad 6 smd rect (at -3.8 1.16 180) (size 0.2 1.5) (layers B.Cu B.Paste B.Mask) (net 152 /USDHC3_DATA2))
  (pad 35 smd rect (at 4.2 -1.16 180) (size 0.2 1.5) (layers B.Cu B.Paste B.Mask) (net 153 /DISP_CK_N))
  (pad 5 smd rect (at -4.2 1.16 180) (size 0.2 1.5) (layers B.Cu B.Paste B.Mask) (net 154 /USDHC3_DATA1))
  (pad 4 smd rect (at -4.6 1.16 180) (size 0.2 1.5) (layers B.Cu B.Paste B.Mask) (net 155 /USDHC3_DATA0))
  (pad 3 smd rect (at -5 1.16 180) (size 0.2 1.5) (layers B.Cu B.Paste B.Mask) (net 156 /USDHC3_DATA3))
  (pad 2 smd rect (at -5.4 1.16 180) (size 0.2 1.5) (layers B.Cu B.Paste B.Mask) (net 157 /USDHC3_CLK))
  (pad 1 smd rect (at -5.8 1.16 180) (size 0.2 1.5) (layers B.Cu B.Paste B.Mask) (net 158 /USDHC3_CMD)))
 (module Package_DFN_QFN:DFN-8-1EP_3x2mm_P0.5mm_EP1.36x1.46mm (layer B.Cu) (at 169 74.5 90)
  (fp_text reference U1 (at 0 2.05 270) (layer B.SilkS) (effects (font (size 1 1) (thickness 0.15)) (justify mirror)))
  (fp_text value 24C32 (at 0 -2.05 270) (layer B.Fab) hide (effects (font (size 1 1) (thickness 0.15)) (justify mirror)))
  (pad "" smd rect (at 0.325 -0.375 90) (size 0.5 0.6) (layers B.Paste))
  (pad "" smd rect (at 0.325 0.375 90) (size 0.5 0.6) (layers B.Paste))
  (pad "" smd rect (at -0.325 -0.375 90) (size 0.5 0.6) (layers B.Paste))
  (pad "" smd rect (at -0.325 0.375 90) (size 0.5 0.6) (layers B.Paste))
  (pad 9 smd rect (at 0 0 90) (size 1.36 1.46) (layers B.Cu B.Mask))
  (pad 8 smd rect (at 1.5 0.75 90) (size 0.75 0.3) (layers B.Cu B.Paste B.Mask) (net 85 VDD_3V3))
  (pad 7 smd rect (at 1.5 0.25 90) (size 0.75 0.3) (layers B.Cu B.Paste B.Mask) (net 28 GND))
  (pad 6 smd rect (at 1.5 -0.25 90) (size 0.75 0.3) (layers B.Cu B.Paste B.Mask) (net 142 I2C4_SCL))
  (pad 5 smd rect (at 1.5 -0.75 90) (size 0.75 0.3) (layers B.Cu B.Paste B.Mask) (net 144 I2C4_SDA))
  (pad 4 smd rect (at -1.5 -0.75 90) (size 0.75 0.3) (layers B.Cu B.Paste B.Mask) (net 28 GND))
  (pad 3 smd rect (at -1.5 -0.25 90) (size 0.75 0.3) (layers B.Cu B.Paste B.Mask) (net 85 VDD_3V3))
  (pad 2 smd rect (at -1.5 0.25 90) (size 0.75 0.3) (layers B.Cu B.Paste B.Mask) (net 85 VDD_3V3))
  (pad 1 smd rect (at -1.5 0.75 90) (size 0.75 0.3) (layers B.Cu B.Paste B.Mask) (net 85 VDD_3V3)))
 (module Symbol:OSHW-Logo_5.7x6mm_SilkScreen (layer B.Cu) (at 111.5 99 180)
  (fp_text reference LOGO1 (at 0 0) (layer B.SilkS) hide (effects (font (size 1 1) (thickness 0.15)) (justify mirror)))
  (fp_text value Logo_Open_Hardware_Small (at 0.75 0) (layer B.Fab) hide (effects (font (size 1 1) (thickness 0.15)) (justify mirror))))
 (gr_line (start 71 138) (end 71 86) (layer Edge.Cuts) (width 0.15))
 (gr_line (start 75 86) (end 71 86) (layer Edge.Cuts) (width 0.15))
 (gr_line (start 75 138) (end 75 86) (layer Edge.Cuts) (width 0.15))
 (gr_line (start 71 138) (end 75 138) (layer Edge.Cuts) (width 0.15))
 (gr_arc (start 197.928932 154.999999) (end 201.464466 151.464466) (angle -45) (layer Edge.Cuts) (width 0.2))
 (gr_line (start 72.071067 150) (end 197.928932 150) (layer Edge.Cuts) (width 0.2))
 (gr_arc (start 72.071067 154.999999) (end 72.071067 150) (angle -45) (layer Edge.Cuts) (width 0.2))
 (gr_line (start 66.802573 153.197426) (end 68.535533 151.464466) (layer Edge.Cuts) (width 0.2))
 (gr_arc (start 63.267039 149.661892) (end 63.267039 154.661892) (angle -45) (layer Edge.Cuts) (width 0.2))
 (gr_line (start 35.338107 154.661892) (end 63.267039 154.661892) (layer Edge.Cuts) (width 0.2))
 (gr_arc (start 35.338107 149.661892) (end 30.338107 149.661892) (angle -90) (layer Edge.Cuts) (width 0.2))
 (gr_line (start 30.338107 70.338108) (end 30.338107 149.661892) (layer Edge.Cuts) (width 0.2))
 (gr_arc (start 35.338107 70.338108) (end 35.338107 65.338108) (angle -90) (layer Edge.Cuts) (width 0.2))
 (gr_line (start 63.267039 65.338108) (end 35.338107 65.338108) (layer Edge.Cuts) (width 0.2))
 (gr_arc (start 63.267039 70.338108) (end 66.802573 66.802574) (angle -45) (layer Edge.Cuts) (width 0.2))
 (gr_line (start 68.535533 68.535534) (end 66.802573 66.802574) (layer Edge.Cuts) (width 0.2))
 (gr_arc (start 72.071067 65.000001) (end 68.535533 68.535534) (angle -45) (layer Edge.Cuts) (width 0.2))
 (gr_line (start 72.071067 70) (end 197.928932 70) (layer Edge.Cuts) (width 0.2))
 (gr_arc (start 197.928932 65) (end 197.928932 70) (angle -45) (layer Edge.Cuts) (width 0.2))
 (gr_line (start 201.464466 68.535534) (end 203.197426 66.802574) (layer Edge.Cuts) (width 0.2))
 (gr_arc (start 206.73296 70.338108) (end 206.73296 65.338108) (angle -45) (layer Edge.Cuts) (width 0.2))
 (gr_line (start 206.73296 65.338108) (end 234.661892 65.338108) (layer Edge.Cuts) (width 0.2))
 (gr_arc (start 234.661892 70.338108) (end 239.661892 70.338108) (angle -90) (layer Edge.Cuts) (width 0.2))
 (gr_line (start 239.661892 70.338108) (end 239.661892 149.661892) (layer Edge.Cuts) (width 0.2))
 (gr_arc (start 234.661892 149.661892) (end 234.661892 154.661892) (angle -90) (layer Edge.Cuts) (width 0.2))
 (gr_line (start 234.661892 154.661892) (end 206.73296 154.661892) (layer Edge.Cuts) (width 0.2))
 (gr_arc (start 206.73296 149.661892) (end 203.197426 153.197426) (angle -45) (layer Edge.Cuts) (width 0.2))
 (gr_line (start 203.197426 153.197426) (end 201.464466 151.464466) (layer Edge.Cuts) (width 0.2))
 (via (at 169.75 72.2) (size 0.4572) (drill 0.254) (layers F.Cu B.Cu) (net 85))
 (segment (start 169.75 73) (end 169.75 72.2) (width 0.254) (layer B.Cu) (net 85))
 (via (at 169.75 77.05) (size 0.4572) (drill 0.254) (layers F.Cu B.Cu) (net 85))
 (segment (start 169.75 76) (end 169.75 77.05) (width 0.254) (layer B.Cu) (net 85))
 (segment (start 169.25 76) (end 169.25 77.05) (width 0.254) (layer B.Cu) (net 85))
 (segment (start 169.25 77.05) (end 169.75 77.05) (width 0.254) (layer B.Cu) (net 85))
 (segment (start 168.75 77.05) (end 169.25 77.05) (width 0.254) (layer B.Cu) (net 85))
 (segment (start 168.75 76) (end 168.75 77.05) (width 0.254) (layer B.Cu) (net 85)))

